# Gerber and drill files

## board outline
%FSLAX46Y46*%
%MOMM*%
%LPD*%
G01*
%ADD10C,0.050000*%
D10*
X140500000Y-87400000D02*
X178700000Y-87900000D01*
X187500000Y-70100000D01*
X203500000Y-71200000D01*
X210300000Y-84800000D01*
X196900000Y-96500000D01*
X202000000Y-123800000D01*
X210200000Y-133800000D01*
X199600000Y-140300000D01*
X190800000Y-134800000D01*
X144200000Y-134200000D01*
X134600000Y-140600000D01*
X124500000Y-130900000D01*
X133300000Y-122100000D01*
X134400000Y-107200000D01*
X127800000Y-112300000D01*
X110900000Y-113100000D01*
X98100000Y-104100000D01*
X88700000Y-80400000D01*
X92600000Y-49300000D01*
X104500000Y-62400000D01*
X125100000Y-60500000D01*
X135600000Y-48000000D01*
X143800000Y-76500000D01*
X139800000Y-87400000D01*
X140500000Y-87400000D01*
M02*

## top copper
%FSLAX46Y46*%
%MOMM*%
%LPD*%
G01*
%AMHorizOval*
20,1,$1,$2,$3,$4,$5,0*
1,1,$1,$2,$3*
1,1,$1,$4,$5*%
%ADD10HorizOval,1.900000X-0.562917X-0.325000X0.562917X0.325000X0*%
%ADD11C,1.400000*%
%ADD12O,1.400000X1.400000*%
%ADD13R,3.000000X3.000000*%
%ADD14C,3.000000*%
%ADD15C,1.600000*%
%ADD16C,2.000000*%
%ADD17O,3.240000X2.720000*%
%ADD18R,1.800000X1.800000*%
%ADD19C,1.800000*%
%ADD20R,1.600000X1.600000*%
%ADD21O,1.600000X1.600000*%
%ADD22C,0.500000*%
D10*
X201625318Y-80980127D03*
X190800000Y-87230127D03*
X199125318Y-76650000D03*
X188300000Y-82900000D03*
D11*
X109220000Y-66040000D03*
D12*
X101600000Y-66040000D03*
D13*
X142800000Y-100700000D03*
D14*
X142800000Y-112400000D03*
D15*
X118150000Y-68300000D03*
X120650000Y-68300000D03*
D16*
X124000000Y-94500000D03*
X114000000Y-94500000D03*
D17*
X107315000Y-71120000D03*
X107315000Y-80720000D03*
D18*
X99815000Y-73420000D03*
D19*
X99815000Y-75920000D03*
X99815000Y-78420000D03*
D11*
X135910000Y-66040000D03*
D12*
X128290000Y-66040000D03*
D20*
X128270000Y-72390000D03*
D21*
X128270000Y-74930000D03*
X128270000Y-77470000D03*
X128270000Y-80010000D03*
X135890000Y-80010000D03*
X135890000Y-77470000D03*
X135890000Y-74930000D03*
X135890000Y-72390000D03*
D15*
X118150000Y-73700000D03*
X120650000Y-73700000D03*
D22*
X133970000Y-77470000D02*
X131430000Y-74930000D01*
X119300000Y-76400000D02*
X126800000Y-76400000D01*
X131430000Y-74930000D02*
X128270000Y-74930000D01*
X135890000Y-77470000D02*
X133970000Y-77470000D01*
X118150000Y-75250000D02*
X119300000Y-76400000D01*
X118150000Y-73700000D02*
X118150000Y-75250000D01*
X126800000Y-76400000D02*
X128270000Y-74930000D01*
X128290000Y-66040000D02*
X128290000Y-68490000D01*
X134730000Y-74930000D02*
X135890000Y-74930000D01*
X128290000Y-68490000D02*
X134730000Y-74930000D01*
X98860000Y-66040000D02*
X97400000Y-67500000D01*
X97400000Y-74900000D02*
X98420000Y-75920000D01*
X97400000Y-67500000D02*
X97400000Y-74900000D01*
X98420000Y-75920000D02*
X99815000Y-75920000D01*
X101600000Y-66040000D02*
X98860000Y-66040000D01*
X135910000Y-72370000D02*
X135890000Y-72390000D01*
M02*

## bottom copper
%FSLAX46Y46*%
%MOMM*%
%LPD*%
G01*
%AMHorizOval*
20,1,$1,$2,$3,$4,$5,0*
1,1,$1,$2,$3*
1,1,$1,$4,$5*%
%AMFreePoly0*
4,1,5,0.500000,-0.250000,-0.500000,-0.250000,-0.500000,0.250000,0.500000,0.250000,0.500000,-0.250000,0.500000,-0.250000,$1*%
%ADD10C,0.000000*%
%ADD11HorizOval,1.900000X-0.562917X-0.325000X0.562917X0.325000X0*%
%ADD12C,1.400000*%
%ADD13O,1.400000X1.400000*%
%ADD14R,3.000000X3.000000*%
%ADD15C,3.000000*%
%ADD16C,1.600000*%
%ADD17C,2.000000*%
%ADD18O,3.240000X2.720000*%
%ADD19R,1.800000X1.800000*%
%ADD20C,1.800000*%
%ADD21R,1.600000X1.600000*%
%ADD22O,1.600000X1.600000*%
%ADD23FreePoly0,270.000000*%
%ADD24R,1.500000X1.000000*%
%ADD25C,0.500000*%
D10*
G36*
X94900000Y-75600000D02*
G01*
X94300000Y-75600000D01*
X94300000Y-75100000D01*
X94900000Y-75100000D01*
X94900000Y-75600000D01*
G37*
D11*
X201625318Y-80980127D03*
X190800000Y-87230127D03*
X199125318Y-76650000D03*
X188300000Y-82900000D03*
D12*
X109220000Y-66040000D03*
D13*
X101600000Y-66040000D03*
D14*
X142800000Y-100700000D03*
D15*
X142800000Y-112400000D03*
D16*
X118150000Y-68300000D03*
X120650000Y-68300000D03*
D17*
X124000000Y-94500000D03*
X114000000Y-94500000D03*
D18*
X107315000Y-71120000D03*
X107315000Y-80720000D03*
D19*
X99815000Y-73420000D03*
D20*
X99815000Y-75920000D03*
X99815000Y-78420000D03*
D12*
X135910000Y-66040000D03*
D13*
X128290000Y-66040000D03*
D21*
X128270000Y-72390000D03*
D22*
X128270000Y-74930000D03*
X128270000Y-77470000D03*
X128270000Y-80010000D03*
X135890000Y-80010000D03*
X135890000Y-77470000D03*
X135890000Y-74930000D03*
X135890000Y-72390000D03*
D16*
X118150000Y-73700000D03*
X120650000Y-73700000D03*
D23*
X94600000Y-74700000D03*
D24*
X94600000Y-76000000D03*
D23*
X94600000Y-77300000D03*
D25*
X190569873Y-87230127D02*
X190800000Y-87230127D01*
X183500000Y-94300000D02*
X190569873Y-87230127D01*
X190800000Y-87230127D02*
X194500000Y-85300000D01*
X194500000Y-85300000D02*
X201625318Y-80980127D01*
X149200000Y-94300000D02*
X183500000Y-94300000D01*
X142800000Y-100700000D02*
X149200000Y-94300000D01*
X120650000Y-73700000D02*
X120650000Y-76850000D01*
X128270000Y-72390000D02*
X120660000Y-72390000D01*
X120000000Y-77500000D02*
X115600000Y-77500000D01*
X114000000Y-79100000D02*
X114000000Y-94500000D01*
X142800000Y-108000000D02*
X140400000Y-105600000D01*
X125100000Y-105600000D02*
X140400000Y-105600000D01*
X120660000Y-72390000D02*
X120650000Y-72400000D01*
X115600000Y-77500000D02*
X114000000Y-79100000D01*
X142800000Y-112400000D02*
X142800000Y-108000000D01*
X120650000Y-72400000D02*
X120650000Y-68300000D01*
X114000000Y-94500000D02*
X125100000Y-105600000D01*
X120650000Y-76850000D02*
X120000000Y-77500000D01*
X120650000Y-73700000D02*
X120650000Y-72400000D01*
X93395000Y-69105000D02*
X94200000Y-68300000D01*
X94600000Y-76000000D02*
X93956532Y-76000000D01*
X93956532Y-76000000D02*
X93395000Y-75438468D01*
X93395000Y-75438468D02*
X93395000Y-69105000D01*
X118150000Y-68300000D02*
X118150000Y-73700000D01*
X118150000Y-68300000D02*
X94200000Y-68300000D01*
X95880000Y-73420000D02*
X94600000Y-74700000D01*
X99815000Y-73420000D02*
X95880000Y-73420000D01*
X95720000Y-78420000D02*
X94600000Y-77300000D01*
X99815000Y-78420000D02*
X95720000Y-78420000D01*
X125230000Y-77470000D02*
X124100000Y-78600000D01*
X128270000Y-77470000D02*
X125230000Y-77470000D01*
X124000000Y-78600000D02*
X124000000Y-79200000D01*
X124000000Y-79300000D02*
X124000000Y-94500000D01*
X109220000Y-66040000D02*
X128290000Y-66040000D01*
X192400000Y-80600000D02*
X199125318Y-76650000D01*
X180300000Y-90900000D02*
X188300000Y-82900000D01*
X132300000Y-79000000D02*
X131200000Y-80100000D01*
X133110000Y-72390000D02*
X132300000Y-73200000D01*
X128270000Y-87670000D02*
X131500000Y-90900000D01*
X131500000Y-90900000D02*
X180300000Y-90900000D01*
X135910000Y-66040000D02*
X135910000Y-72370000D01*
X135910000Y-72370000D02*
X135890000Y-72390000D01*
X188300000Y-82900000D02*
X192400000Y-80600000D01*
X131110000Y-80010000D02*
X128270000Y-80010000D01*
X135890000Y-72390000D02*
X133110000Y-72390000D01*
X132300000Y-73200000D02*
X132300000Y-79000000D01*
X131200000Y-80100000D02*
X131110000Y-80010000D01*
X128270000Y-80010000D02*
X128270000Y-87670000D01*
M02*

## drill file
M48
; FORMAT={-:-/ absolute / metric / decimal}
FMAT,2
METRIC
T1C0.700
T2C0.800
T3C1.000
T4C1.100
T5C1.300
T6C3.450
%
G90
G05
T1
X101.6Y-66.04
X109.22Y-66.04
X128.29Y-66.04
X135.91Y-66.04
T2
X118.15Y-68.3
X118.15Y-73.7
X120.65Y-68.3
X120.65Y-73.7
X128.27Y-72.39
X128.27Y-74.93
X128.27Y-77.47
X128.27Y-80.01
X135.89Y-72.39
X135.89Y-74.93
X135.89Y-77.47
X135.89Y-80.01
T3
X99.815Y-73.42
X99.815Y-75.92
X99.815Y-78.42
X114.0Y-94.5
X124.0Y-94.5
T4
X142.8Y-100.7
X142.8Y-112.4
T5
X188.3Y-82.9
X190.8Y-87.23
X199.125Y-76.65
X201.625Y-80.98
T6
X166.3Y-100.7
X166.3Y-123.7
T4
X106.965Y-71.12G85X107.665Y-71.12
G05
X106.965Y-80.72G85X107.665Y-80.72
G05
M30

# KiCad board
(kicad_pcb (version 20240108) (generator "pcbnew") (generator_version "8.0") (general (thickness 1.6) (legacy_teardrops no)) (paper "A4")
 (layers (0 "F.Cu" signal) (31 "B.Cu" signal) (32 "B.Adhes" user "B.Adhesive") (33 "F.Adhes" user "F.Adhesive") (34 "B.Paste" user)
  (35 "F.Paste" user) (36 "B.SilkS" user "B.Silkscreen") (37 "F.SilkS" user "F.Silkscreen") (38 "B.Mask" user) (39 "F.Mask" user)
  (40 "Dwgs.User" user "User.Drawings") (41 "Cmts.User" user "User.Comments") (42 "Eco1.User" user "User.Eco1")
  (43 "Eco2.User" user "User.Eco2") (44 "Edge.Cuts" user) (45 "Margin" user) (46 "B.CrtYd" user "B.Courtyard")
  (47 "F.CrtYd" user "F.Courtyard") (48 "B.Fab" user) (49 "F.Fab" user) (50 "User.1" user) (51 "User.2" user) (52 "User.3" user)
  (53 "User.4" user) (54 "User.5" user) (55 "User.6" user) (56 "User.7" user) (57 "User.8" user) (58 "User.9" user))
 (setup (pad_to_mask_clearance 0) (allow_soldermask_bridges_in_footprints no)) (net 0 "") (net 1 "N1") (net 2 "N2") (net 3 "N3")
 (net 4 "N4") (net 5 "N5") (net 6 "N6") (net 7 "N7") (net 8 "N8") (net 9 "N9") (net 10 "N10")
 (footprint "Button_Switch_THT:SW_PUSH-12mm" (layer "F.Cu") (at 201.625318 80.980127 -150)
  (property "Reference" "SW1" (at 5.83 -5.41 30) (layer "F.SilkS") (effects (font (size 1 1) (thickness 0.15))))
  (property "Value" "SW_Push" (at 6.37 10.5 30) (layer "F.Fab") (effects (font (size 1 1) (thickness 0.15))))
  (pad "1" thru_hole oval (at 0 0 210) (size 3.2 1.9) (drill 1.3) (layers "*.Cu" "*.Mask") (remove_unused_layers no) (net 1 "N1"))
  (pad "1" thru_hole oval (at 12.5 0 210) (size 3.2 1.9) (drill 1.3) (layers "*.Cu" "*.Mask") (remove_unused_layers no) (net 1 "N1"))
  (pad "2" thru_hole oval (at 0 5 210) (size 3.2 1.9) (drill 1.3) (layers "*.Cu" "*.Mask") (remove_unused_layers no) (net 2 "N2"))
  (pad "2" thru_hole oval (at 12.5 5 210) (size 3.2 1.9) (drill 1.3) (layers "*.Cu" "*.Mask") (remove_unused_layers no) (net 2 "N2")))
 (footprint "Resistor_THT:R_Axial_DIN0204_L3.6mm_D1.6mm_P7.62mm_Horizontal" (layer "F.Cu") (at 109.22 66.04 180)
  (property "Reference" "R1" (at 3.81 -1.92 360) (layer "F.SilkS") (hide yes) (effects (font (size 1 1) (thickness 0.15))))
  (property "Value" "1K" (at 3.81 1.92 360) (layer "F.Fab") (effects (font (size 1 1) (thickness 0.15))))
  (pad "1" thru_hole circle (at 0 0 180) (size 1.4 1.4) (drill 0.7) (layers "*.Cu" "*.Mask") (remove_unused_layers no) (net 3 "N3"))
  (pad "2" thru_hole oval (at 7.62 0 180) (size 1.4 1.4) (drill 0.7) (layers "*.Cu" "*.Mask") (remove_unused_layers no) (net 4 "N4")))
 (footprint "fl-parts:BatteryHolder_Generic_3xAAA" (layer "F.Cu") (at 140.3 94.2)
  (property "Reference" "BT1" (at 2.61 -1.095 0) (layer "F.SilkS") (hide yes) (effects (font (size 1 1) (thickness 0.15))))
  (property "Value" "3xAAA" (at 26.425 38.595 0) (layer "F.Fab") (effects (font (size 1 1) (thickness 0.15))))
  (pad "" np_thru_hole circle (at 26 6.5) (size 3.45 3.45) (drill 3.45) (layers "F&B.Cu" "*.Mask"))
  (pad "" np_thru_hole circle (at 26 29.5) (size 3.45 3.45) (drill 3.45) (layers "F&B.Cu" "*.Mask"))
  (pad "1" thru_hole rect (at 2.5 6.5) (size 3 3) (drill 1.1) (layers "*.Cu" "*.Mask") (remove_unused_layers no) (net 1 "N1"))
  (pad "2" thru_hole circle (at 2.5 18.2) (size 3 3) (drill 1.1) (layers "*.Cu" "*.Mask") (remove_unused_layers no) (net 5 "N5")))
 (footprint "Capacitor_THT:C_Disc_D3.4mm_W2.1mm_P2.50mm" (layer "F.Cu") (at 118.15 68.3)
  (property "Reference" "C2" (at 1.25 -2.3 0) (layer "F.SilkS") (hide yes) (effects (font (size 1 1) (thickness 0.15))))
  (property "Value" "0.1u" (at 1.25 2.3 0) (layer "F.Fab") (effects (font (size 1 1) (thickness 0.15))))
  (pad "1" thru_hole circle (at 0 0) (size 1.6 1.6) (drill 0.8) (layers "*.Cu" "*.Mask") (remove_unused_layers no) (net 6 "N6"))
  (pad "2" thru_hole circle (at 2.5 0) (size 1.6 1.6) (drill 0.8) (layers "*.Cu" "*.Mask") (remove_unused_layers no) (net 5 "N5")))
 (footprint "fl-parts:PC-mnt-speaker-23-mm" (layer "F.Cu") (at 119 94.5 180)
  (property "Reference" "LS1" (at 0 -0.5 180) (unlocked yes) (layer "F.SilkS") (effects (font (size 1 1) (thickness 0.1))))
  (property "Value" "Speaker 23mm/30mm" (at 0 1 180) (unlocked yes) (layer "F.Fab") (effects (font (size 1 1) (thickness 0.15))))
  (pad "1" thru_hole circle (at -5 0 180) (size 2 2) (drill 1) (layers "*.Cu" "*.Mask") (remove_unused_layers no) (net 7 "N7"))
  (pad "2" thru_hole circle (at 5 0 180) (size 2 2) (drill 1) (layers "*.Cu" "*.Mask") (remove_unused_layers no) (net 5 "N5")))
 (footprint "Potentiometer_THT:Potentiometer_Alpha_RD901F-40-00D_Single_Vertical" (layer "F.Cu") (at 99.815 73.42)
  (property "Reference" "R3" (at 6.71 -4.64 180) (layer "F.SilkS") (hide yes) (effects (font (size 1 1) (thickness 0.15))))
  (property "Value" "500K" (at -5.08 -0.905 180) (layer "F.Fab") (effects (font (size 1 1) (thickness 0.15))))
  (pad "" thru_hole oval (at 7.5 -2.3 90) (size 2.72 3.24) (drill oval 1.1 1.8) (layers "*.Cu" "*.Mask") (remove_unused_layers no))
  (pad "" thru_hole oval (at 7.5 7.3 90) (size 2.72 3.24) (drill oval 1.1 1.8) (layers "*.Cu" "*.Mask") (remove_unused_layers no))
  (pad "1" thru_hole rect (at 0 0 90) (size 1.8 1.8) (drill 1) (layers "*.Cu" "*.Mask") (remove_unused_layers no) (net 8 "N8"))
  (pad "2" thru_hole circle (at 0 2.5 90) (size 1.8 1.8) (drill 1) (layers "*.Cu" "*.Mask") (remove_unused_layers no) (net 4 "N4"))
  (pad "3" thru_hole circle (at 0 5 90) (size 1.8 1.8) (drill 1) (layers "*.Cu" "*.Mask") (remove_unused_layers no) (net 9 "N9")))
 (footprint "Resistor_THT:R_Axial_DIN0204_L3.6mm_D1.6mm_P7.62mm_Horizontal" (layer "F.Cu") (at 135.91 66.04 180)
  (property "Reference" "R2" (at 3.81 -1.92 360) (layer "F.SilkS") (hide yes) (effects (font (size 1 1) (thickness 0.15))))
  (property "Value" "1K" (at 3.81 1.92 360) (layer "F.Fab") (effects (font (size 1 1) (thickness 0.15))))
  (pad "1" thru_hole circle (at 0 0 180) (size 1.4 1.4) (drill 0.7) (layers "*.Cu" "*.Mask") (remove_unused_layers no) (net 2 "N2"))
  (pad "2" thru_hole oval (at 7.62 0 180) (size 1.4 1.4) (drill 0.7) (layers "*.Cu" "*.Mask") (remove_unused_layers no) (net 3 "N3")))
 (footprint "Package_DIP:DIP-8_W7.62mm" (layer "F.Cu") (at 128.27 72.39)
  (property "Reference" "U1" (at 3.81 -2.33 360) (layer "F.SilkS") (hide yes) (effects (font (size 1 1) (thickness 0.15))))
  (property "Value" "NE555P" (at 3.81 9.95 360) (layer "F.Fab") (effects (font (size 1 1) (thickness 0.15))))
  (pad "1" thru_hole rect (at 0 0) (size 1.6 1.6) (drill 0.8) (layers "*.Cu" "*.Mask") (remove_unused_layers no) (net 5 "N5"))
  (pad "2" thru_hole oval (at 0 2.54) (size 1.6 1.6) (drill 0.8) (layers "*.Cu" "*.Mask") (remove_unused_layers no) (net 6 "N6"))
  (pad "3" thru_hole oval (at 0 5.08) (size 1.6 1.6) (drill 0.8) (layers "*.Cu" "*.Mask") (remove_unused_layers no) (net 7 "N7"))
  (pad "4" thru_hole oval (at 0 7.62) (size 1.6 1.6) (drill 0.8) (layers "*.Cu" "*.Mask") (remove_unused_layers no) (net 2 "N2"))
  (pad "5" thru_hole oval (at 7.62 7.62) (size 1.6 1.6) (drill 0.8) (layers "*.Cu" "*.Mask") (remove_unused_layers no) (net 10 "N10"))
  (pad "6" thru_hole oval (at 7.62 5.08) (size 1.6 1.6) (drill 0.8) (layers "*.Cu" "*.Mask") (remove_unused_layers no) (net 6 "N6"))
  (pad "7" thru_hole oval (at 7.62 2.54) (size 1.6 1.6) (drill 0.8) (layers "*.Cu" "*.Mask") (remove_unused_layers no) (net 3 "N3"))
  (pad "8" thru_hole oval (at 7.62 0) (size 1.6 1.6) (drill 0.8) (layers "*.Cu" "*.Mask") (remove_unused_layers no) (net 2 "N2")))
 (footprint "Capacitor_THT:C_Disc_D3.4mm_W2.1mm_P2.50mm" (layer "F.Cu") (at 118.15 73.7)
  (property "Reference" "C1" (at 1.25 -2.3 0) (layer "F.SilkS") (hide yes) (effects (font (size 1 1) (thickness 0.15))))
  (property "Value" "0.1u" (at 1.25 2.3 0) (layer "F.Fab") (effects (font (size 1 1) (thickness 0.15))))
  (pad "1" thru_hole circle (at 0 0) (size 1.6 1.6) (drill 0.8) (layers "*.Cu" "*.Mask") (remove_unused_layers no) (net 6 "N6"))
  (pad "2" thru_hole circle (at 2.5 0) (size 1.6 1.6) (drill 0.8) (layers "*.Cu" "*.Mask") (remove_unused_layers no) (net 5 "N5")))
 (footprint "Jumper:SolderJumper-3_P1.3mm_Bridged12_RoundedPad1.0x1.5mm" (layer "B.Cu") (at 94.6 76 -90)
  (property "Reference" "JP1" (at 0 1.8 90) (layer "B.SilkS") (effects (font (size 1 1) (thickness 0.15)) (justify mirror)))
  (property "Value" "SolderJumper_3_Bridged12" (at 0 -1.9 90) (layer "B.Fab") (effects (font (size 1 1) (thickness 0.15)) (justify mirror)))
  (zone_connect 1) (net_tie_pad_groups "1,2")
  (fp_poly (pts (xy -0.9 0.3) (xy -0.4 0.3) (xy -0.4 -0.3) (xy -0.9 -0.3)) (stroke (width 0) (type solid)) (fill solid) (layer "B.Cu"))
  (pad "1" smd custom (at -1.3 0 270) (size 1 0.5) (layers "B.Cu" "B.Mask") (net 8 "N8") (zone_connect 2) (thermal_bridge_angle 45)
   (options (clearance outline) (anchor rect)) (primitives))
  (pad "2" smd rect (at 0 0 270) (size 1 1.5) (layers "B.Cu" "B.Mask") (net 6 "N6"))
  (pad "3" smd custom (at 1.3 0 270) (size 1 0.5) (layers "B.Cu" "B.Mask") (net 9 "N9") (zone_connect 2) (thermal_bridge_angle 45)
   (options (clearance outline) (anchor rect)) (primitives)))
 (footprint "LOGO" (layer "B.Cu") (at 180.9 119.6 180)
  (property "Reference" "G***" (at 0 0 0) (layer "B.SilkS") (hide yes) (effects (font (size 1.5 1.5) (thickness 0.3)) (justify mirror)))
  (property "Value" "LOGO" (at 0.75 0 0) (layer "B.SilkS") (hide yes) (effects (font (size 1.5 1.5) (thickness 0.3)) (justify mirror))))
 (gr_poly
  (pts (xy 140.5 87.4) (xy 178.7 87.9) (xy 187.5 70.1) (xy 203.5 71.2) (xy 210.3 84.8) (xy 196.9 96.5) (xy 202 123.8) (xy 210.2 133.8)
   (xy 199.6 140.3) (xy 190.8 134.8) (xy 144.2 134.2) (xy 134.6 140.6) (xy 124.5 130.9) (xy 133.3 122.1) (xy 134.4 107.2) (xy 127.8 112.3)
   (xy 110.9 113.1) (xy 98.1 104.1) (xy 88.7 80.4) (xy 92.6 49.3) (xy 104.5 62.4) (xy 125.1 60.5) (xy 135.6 48) (xy 143.8 76.5)
   (xy 139.8 87.4) (xy 139.8 87.4) (xy 140.5 87.4) (xy 140.5 87.4))
  (stroke (width 0.05) (type solid)) (fill none) (layer "Edge.Cuts"))
 (segment (start 190.569873 87.230127) (end 190.8 87.230127) (width 0.5) (layer "B.Cu") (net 1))
 (segment (start 183.5 94.3) (end 190.569873 87.230127) (width 0.5) (layer "B.Cu") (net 1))
 (segment (start 190.8 87.230127) (end 194.5 85.3) (width 0.5) (layer "B.Cu") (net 1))
 (segment (start 194.5 85.3) (end 201.625318 80.980127) (width 0.5) (layer "B.Cu") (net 1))
 (segment (start 149.2 94.3) (end 183.5 94.3) (width 0.5) (layer "B.Cu") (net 1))
 (segment (start 142.8 100.7) (end 149.2 94.3) (width 0.5) (layer "B.Cu") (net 1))
 (segment (start 120.65 73.7) (end 120.65 76.85) (width 0.5) (layer "B.Cu") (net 5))
 (segment (start 128.27 72.39) (end 120.66 72.39) (width 0.5) (layer "B.Cu") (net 5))
 (segment (start 120 77.5) (end 115.6 77.5) (width 0.5) (layer "B.Cu") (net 5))
 (segment (start 114 79.1) (end 114 94.5) (width 0.5) (layer "B.Cu") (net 5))
 (segment (start 142.8 108) (end 140.4 105.6) (width 0.5) (layer "B.Cu") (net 5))
 (segment (start 125.1 105.6) (end 140.4 105.6) (width 0.5) (layer "B.Cu") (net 5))
 (segment (start 120.66 72.39) (end 120.65 72.4) (width 0.5) (layer "B.Cu") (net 5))
 (segment (start 115.6 77.5) (end 114 79.1) (width 0.5) (layer "B.Cu") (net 5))
 (segment (start 142.8 112.4) (end 142.8 108) (width 0.5) (layer "B.Cu") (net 5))
 (segment (start 120.65 72.4) (end 120.65 68.3) (width 0.5) (layer "B.Cu") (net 5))
 (segment (start 114 94.5) (end 125.1 105.6) (width 0.5) (layer "B.Cu") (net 5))
 (segment (start 120.65 76.85) (end 120 77.5) (width 0.5) (layer "B.Cu") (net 5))
 (segment (start 120.65 73.7) (end 120.65 72.4) (width 0.5) (layer "B.Cu") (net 5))
 (segment (start 133.97 77.47) (end 131.43 74.93) (width 0.5) (layer "F.Cu") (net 6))
 (segment (start 119.3 76.4) (end 126.8 76.4) (width 0.5) (layer "F.Cu") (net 6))
 (segment (start 131.43 74.93) (end 128.27 74.93) (width 0.5) (layer "F.Cu") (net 6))
 (segment (start 135.89 77.47) (end 133.97 77.47) (width 0.5) (layer "F.Cu") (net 6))
 (segment (start 118.15 75.25) (end 119.3 76.4) (width 0.5) (layer "F.Cu") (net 6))
 (segment (start 118.15 73.7) (end 118.15 75.25) (width 0.5) (layer "F.Cu") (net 6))
 (segment (start 126.8 76.4) (end 128.27 74.93) (width 0.5) (layer "F.Cu") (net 6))
 (segment (start 93.395 69.105) (end 94.2 68.3) (width 0.5) (layer "B.Cu") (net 6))
 (segment (start 94.6 76) (end 93.956532 76) (width 0.5) (layer "B.Cu") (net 6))
 (segment (start 93.956532 76) (end 93.395 75.438468) (width 0.5) (layer "B.Cu") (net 6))
 (segment (start 93.395 75.438468) (end 93.395 69.105) (width 0.5) (layer "B.Cu") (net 6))
 (segment (start 118.15 68.3) (end 118.15 73.7) (width 0.5) (layer "B.Cu") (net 6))
 (segment (start 118.15 68.3) (end 94.2 68.3) (width 0.5) (layer "B.Cu") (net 6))
 (segment (start 95.88 73.42) (end 94.6 74.7) (width 0.5) (layer "B.Cu") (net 8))
 (segment (start 99.815 73.42) (end 95.88 73.42) (width 0.5) (layer "B.Cu") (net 8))
 (segment (start 95.72 78.42) (end 94.6 77.3) (width 0.5) (layer "B.Cu") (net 9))
 (segment (start 99.815 78.42) (end 95.72 78.42) (width 0.5) (layer "B.Cu") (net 9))
 (segment (start 125.23 77.47) (end 124.1 78.6) (width 0.5) (layer "B.Cu") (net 7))
 (segment (start 128.27 77.47) (end 125.23 77.47) (width 0.5) (layer "B.Cu") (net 7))
 (segment (start 124 78.6) (end 124 79.2) (width 0.5) (layer "B.Cu") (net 7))
 (segment (start 124 79.3) (end 124 94.5) (width 0.5) (layer "B.Cu") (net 7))
 (segment (start 128.29 66.04) (end 128.29 68.49) (width 0.5) (layer "F.Cu") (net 3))
 (segment (start 134.73 74.93) (end 135.89 74.93) (width 0.5) (layer "F.Cu") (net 3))
 (segment (start 128.29 68.49) (end 134.73 74.93) (width 0.5) (layer "F.Cu") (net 3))
 (segment (start 109.22 66.04) (end 128.29 66.04) (width 0.5) (layer "B.Cu") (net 3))
 (segment (start 98.86 66.04) (end 97.4 67.5) (width 0.5) (layer "F.Cu") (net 4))
 (segment (start 97.4 74.9) (end 98.42 75.92) (width 0.5) (layer "F.Cu") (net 4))
 (segment (start 97.4 67.5) (end 97.4 74.9) (width 0.5) (layer "F.Cu") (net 4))
 (segment (start 98.42 75.92) (end 99.815 75.92) (width 0.5) (layer "F.Cu") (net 4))
 (segment (start 101.6 66.04) (end 98.86 66.04) (width 0.5) (layer "F.Cu") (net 4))
 (segment (start 135.91 72.37) (end 135.89 72.39) (width 0.5) (layer "F.Cu") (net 2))
 (segment (start 192.4 80.6) (end 199.125318 76.65) (width 0.5) (layer "B.Cu") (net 2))
 (segment (start 180.3 90.9) (end 188.3 82.9) (width 0.5) (layer "B.Cu") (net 2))
 (segment (start 132.3 79) (end 131.2 80.1) (width 0.5) (layer "B.Cu") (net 2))
 (segment (start 133.11 72.39) (end 132.3 73.2) (width 0.5) (layer "B.Cu") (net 2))
 (segment (start 128.27 87.67) (end 131.5 90.9) (width 0.5) (layer "B.Cu") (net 2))
 (segment (start 131.5 90.9) (end 180.3 90.9) (width 0.5) (layer "B.Cu") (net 2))
 (segment (start 135.91 66.04) (end 135.91 72.37) (width 0.5) (layer "B.Cu") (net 2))
 (segment (start 135.91 72.37) (end 135.89 72.39) (width 0.5) (layer "B.Cu") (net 2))
 (segment (start 188.3 82.9) (end 192.4 80.6) (width 0.5) (layer "B.Cu") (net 2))
 (segment (start 131.11 80.01) (end 128.27 80.01) (width 0.5) (layer "B.Cu") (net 2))
 (segment (start 135.89 72.39) (end 133.11 72.39) (width 0.5) (layer "B.Cu") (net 2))
 (segment (start 132.3 73.2) (end 132.3 79) (width 0.5) (layer "B.Cu") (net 2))
 (segment (start 131.2 80.1) (end 131.11 80.01) (width 0.5) (layer "B.Cu") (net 2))
 (segment (start 128.27 80.01) (end 128.27 87.67) (width 0.5) (layer "B.Cu") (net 2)))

